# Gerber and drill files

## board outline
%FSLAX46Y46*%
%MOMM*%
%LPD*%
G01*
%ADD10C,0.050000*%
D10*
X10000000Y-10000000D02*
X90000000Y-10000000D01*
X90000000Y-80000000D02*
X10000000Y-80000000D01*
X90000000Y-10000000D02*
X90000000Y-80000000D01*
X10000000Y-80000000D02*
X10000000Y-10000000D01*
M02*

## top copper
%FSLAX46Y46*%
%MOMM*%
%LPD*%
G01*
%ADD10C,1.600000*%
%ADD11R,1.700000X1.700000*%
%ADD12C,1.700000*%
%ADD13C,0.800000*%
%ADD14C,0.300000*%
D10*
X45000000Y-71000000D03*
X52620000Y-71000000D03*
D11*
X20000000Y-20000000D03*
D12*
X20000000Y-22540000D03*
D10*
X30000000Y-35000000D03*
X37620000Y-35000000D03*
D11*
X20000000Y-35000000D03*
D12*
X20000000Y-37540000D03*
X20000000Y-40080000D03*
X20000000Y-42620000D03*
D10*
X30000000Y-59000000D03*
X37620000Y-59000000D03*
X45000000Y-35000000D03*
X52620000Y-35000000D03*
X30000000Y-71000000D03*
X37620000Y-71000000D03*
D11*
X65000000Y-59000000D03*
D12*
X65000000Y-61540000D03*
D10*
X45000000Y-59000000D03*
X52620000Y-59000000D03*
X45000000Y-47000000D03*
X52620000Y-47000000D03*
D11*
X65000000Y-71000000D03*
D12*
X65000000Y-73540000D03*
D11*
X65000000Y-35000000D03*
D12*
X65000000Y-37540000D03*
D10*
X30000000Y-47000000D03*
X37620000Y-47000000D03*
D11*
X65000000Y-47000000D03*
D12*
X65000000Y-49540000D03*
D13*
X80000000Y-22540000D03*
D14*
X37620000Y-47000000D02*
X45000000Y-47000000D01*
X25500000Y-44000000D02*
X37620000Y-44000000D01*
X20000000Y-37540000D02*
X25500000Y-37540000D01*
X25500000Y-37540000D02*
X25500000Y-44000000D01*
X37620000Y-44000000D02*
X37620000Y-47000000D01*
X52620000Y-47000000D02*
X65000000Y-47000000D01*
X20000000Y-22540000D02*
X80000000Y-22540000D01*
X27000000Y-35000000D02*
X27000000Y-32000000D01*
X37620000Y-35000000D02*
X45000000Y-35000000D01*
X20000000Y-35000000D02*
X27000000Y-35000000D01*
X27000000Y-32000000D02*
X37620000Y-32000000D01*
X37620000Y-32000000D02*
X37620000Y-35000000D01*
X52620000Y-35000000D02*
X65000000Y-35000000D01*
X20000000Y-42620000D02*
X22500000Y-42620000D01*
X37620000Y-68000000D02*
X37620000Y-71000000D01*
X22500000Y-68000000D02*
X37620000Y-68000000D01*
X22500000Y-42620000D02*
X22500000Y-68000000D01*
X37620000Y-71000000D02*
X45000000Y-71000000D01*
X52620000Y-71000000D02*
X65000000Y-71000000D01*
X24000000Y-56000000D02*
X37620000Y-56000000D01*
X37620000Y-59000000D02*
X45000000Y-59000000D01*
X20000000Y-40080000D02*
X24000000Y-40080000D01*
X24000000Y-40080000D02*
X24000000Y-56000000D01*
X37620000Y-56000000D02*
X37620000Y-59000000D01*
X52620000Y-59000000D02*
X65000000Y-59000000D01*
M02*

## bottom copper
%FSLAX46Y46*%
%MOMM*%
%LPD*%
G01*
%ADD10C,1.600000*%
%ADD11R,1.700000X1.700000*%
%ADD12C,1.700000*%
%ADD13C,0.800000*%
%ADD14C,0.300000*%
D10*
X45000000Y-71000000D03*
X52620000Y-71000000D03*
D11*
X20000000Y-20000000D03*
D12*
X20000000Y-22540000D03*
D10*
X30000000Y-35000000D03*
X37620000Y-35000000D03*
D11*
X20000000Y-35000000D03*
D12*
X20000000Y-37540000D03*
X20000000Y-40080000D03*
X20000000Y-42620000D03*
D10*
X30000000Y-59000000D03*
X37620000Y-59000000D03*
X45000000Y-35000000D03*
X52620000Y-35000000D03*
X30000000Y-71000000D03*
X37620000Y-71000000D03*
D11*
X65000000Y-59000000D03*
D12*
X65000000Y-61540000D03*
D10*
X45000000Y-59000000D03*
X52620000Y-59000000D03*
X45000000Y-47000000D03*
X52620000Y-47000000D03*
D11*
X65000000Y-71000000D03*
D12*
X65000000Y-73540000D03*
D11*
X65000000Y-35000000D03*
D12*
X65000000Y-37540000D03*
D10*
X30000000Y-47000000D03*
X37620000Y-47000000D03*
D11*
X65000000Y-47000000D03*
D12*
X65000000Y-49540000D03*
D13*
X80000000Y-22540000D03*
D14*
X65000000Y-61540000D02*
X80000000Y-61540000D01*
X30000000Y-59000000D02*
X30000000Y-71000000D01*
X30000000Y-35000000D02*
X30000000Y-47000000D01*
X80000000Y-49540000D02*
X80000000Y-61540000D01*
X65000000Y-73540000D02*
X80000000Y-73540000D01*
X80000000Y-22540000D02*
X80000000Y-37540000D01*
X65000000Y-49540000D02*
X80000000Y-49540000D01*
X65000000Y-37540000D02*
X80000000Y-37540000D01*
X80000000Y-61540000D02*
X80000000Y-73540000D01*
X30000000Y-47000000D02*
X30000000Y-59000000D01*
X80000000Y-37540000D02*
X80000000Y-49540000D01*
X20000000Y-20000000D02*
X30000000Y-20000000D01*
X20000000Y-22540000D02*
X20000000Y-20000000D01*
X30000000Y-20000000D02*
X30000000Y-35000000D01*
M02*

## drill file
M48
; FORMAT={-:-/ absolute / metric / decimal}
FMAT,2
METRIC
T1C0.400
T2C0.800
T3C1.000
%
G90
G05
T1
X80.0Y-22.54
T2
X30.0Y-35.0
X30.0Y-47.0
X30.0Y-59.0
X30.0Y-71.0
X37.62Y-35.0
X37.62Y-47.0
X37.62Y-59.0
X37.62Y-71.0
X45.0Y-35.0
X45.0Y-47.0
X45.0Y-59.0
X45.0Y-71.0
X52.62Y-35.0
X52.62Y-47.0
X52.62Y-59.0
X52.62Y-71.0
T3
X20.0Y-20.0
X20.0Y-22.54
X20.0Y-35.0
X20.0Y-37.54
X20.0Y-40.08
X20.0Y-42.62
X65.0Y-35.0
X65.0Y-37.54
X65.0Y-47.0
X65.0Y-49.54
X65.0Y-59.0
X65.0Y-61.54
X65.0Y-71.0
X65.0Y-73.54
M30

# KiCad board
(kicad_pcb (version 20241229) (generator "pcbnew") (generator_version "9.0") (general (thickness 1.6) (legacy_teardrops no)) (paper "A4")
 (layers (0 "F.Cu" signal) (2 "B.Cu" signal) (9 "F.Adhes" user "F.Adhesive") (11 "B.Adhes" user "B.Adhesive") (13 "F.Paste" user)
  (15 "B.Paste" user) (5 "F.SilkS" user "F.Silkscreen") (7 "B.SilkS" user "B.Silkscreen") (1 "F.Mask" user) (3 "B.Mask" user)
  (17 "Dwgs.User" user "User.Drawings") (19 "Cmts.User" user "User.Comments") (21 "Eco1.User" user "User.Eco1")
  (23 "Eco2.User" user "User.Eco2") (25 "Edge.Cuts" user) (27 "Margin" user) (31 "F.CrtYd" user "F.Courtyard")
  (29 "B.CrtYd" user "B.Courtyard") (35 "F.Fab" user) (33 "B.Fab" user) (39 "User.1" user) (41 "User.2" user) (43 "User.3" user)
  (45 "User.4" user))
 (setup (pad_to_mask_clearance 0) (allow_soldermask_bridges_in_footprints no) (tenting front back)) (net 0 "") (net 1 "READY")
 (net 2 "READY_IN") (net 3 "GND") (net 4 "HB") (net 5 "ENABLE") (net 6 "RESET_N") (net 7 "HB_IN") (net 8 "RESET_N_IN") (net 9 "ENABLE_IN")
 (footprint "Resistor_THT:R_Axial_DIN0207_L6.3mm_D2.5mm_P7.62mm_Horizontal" (layer "F.Cu") (at 45 71)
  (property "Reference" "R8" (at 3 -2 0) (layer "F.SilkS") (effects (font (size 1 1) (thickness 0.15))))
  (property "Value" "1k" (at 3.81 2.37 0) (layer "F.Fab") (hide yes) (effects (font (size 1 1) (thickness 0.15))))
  (pad "1" thru_hole circle (at 0 0) (size 1.6 1.6) (drill 0.8) (layers "*.Cu" "*.Mask") (remove_unused_layers no) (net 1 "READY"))
  (pad "2" thru_hole circle (at 7.62 0) (size 1.6 1.6) (drill 0.8) (layers "*.Cu" "*.Mask") (remove_unused_layers no) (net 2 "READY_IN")))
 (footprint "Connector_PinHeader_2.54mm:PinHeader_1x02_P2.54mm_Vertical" (layer "F.Cu") (at 20 20)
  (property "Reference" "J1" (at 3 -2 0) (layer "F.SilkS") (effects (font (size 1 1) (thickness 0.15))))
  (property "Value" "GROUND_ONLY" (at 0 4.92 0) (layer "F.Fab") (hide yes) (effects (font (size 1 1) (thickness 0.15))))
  (pad "1" thru_hole rect (at 0 0) (size 1.7 1.7) (drill 1) (layers "*.Cu" "*.Mask") (remove_unused_layers no) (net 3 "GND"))
  (pad "2" thru_hole circle (at 0 2.54) (size 1.7 1.7) (drill 1) (layers "*.Cu" "*.Mask") (remove_unused_layers no) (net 3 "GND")))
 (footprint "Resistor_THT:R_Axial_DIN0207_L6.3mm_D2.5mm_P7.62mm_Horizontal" (layer "F.Cu") (at 30 35)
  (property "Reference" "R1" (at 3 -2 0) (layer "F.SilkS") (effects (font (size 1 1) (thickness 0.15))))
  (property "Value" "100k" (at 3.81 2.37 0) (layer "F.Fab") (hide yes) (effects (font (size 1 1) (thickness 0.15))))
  (pad "1" thru_hole circle (at 0 0) (size 1.6 1.6) (drill 0.8) (layers "*.Cu" "*.Mask") (remove_unused_layers no) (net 3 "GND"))
  (pad "2" thru_hole circle (at 7.62 0) (size 1.6 1.6) (drill 0.8) (layers "*.Cu" "*.Mask") (remove_unused_layers no) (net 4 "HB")))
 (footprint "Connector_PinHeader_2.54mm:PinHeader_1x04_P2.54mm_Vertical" (layer "F.Cu") (at 20 35)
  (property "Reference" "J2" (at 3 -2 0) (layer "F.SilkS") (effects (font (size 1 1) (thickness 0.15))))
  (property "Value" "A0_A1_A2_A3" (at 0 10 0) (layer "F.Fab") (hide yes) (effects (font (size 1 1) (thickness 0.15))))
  (pad "1" thru_hole rect (at 0 0) (size 1.7 1.7) (drill 1) (layers "*.Cu" "*.Mask") (remove_unused_layers no) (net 4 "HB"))
  (pad "2" thru_hole circle (at 0 2.54) (size 1.7 1.7) (drill 1) (layers "*.Cu" "*.Mask") (remove_unused_layers no) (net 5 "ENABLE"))
  (pad "3" thru_hole circle (at 0 5.08) (size 1.7 1.7) (drill 1) (layers "*.Cu" "*.Mask") (remove_unused_layers no) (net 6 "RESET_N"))
  (pad "4" thru_hole circle (at 0 7.62) (size 1.7 1.7) (drill 1) (layers "*.Cu" "*.Mask") (remove_unused_layers no) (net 1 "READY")))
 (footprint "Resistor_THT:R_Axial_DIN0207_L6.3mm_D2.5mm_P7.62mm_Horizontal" (layer "F.Cu") (at 30 59)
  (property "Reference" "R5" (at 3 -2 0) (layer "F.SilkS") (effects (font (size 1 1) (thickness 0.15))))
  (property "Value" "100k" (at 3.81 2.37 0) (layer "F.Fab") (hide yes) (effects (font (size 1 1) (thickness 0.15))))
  (pad "1" thru_hole circle (at 0 0) (size 1.6 1.6) (drill 0.8) (layers "*.Cu" "*.Mask") (remove_unused_layers no) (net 3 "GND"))
  (pad "2" thru_hole circle (at 7.62 0) (size 1.6 1.6) (drill 0.8) (layers "*.Cu" "*.Mask") (remove_unused_layers no) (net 6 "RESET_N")))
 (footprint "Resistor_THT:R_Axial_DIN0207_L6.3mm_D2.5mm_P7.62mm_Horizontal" (layer "F.Cu") (at 45 35)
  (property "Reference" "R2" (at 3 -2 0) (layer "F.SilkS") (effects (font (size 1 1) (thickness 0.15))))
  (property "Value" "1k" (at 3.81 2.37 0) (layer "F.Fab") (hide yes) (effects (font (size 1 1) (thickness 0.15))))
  (pad "1" thru_hole circle (at 0 0) (size 1.6 1.6) (drill 0.8) (layers "*.Cu" "*.Mask") (remove_unused_layers no) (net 4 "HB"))
  (pad "2" thru_hole circle (at 7.62 0) (size 1.6 1.6) (drill 0.8) (layers "*.Cu" "*.Mask") (remove_unused_layers no) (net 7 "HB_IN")))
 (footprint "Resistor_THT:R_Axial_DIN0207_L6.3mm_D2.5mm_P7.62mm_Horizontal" (layer "F.Cu") (at 30 71)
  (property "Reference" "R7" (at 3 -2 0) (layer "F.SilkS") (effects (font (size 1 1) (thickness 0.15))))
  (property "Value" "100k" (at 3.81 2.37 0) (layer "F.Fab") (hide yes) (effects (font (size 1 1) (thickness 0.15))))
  (pad "1" thru_hole circle (at 0 0) (size 1.6 1.6) (drill 0.8) (layers "*.Cu" "*.Mask") (remove_unused_layers no) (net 3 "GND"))
  (pad "2" thru_hole circle (at 7.62 0) (size 1.6 1.6) (drill 0.8) (layers "*.Cu" "*.Mask") (remove_unused_layers no) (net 1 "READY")))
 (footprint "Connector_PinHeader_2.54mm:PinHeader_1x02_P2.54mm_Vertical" (layer "F.Cu") (at 65 59)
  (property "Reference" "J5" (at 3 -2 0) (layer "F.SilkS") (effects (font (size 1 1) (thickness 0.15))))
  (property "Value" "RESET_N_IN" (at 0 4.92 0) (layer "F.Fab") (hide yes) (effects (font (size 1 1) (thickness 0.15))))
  (pad "1" thru_hole rect (at 0 0) (size 1.7 1.7) (drill 1) (layers "*.Cu" "*.Mask") (remove_unused_layers no) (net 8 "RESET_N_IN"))
  (pad "2" thru_hole circle (at 0 2.54) (size 1.7 1.7) (drill 1) (layers "*.Cu" "*.Mask") (remove_unused_layers no) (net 3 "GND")))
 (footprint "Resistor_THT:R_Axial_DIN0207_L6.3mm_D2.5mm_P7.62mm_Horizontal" (layer "F.Cu") (at 45 59)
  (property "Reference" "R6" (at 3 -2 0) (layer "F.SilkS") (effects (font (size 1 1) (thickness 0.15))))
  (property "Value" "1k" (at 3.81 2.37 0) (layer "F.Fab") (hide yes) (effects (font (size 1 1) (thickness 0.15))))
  (pad "1" thru_hole circle (at 0 0) (size 1.6 1.6) (drill 0.8) (layers "*.Cu" "*.Mask") (remove_unused_layers no) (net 6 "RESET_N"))
  (pad "2" thru_hole circle (at 7.62 0) (size 1.6 1.6) (drill 0.8) (layers "*.Cu" "*.Mask") (remove_unused_layers no) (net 8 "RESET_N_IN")))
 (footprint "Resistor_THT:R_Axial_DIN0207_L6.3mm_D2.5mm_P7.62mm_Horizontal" (layer "F.Cu") (at 45 47)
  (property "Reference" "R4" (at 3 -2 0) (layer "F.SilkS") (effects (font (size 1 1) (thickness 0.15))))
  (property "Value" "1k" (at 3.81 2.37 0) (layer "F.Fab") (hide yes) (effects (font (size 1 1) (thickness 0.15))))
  (pad "1" thru_hole circle (at 0 0) (size 1.6 1.6) (drill 0.8) (layers "*.Cu" "*.Mask") (remove_unused_layers no) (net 5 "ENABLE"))
  (pad "2" thru_hole circle (at 7.62 0) (size 1.6 1.6) (drill 0.8) (layers "*.Cu" "*.Mask") (remove_unused_layers no) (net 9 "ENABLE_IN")))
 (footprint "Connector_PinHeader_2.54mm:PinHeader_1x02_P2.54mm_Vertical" (layer "F.Cu") (at 65 71)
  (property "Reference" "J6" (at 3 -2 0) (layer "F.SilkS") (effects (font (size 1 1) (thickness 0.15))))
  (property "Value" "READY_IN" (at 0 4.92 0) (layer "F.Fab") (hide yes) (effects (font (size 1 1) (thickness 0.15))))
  (pad "1" thru_hole rect (at 0 0) (size 1.7 1.7) (drill 1) (layers "*.Cu" "*.Mask") (remove_unused_layers no) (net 2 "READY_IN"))
  (pad "2" thru_hole circle (at 0 2.54) (size 1.7 1.7) (drill 1) (layers "*.Cu" "*.Mask") (remove_unused_layers no) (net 3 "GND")))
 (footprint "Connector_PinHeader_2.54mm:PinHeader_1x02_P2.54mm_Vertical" (layer "F.Cu") (at 65 35)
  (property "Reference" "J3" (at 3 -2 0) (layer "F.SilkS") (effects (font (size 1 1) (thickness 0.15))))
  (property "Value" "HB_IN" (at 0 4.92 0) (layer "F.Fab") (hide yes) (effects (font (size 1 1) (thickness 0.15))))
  (pad "1" thru_hole rect (at 0 0) (size 1.7 1.7) (drill 1) (layers "*.Cu" "*.Mask") (remove_unused_layers no) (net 7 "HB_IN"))
  (pad "2" thru_hole circle (at 0 2.54) (size 1.7 1.7) (drill 1) (layers "*.Cu" "*.Mask") (remove_unused_layers no) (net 3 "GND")))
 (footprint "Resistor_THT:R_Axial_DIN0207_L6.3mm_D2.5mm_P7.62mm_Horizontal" (layer "F.Cu") (at 30 47)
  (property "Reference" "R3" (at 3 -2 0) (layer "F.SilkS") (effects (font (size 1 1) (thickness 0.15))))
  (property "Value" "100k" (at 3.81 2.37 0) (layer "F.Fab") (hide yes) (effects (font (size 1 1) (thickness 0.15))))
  (pad "1" thru_hole circle (at 0 0) (size 1.6 1.6) (drill 0.8) (layers "*.Cu" "*.Mask") (remove_unused_layers no) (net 3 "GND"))
  (pad "2" thru_hole circle (at 7.62 0) (size 1.6 1.6) (drill 0.8) (layers "*.Cu" "*.Mask") (remove_unused_layers no) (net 5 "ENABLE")))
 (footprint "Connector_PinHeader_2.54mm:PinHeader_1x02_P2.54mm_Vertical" (layer "F.Cu") (at 65 47)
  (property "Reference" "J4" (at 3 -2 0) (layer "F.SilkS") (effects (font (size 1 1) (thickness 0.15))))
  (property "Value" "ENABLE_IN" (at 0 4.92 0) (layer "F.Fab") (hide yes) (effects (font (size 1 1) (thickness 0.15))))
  (pad "1" thru_hole rect (at 0 0) (size 1.7 1.7) (drill 1) (layers "*.Cu" "*.Mask") (remove_unused_layers no) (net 9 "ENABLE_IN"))
  (pad "2" thru_hole circle (at 0 2.54) (size 1.7 1.7) (drill 1) (layers "*.Cu" "*.Mask") (remove_unused_layers no) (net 3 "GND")))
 (gr_line (start 10 10) (end 90 10) (stroke (width 0.05) (type default)) (layer "Edge.Cuts"))
 (gr_line (start 90 80) (end 10 80) (stroke (width 0.05) (type default)) (layer "Edge.Cuts"))
 (gr_line (start 90 10) (end 90 80) (stroke (width 0.05) (type default)) (layer "Edge.Cuts"))
 (gr_line (start 10 80) (end 10 10) (stroke (width 0.05) (type default)) (layer "Edge.Cuts"))
 (segment (start 37.62 47) (end 45 47) (width 0.3) (layer "F.Cu") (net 5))
 (segment (start 25.5 44) (end 37.62 44) (width 0.3) (layer "F.Cu") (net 5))
 (segment (start 20 37.54) (end 25.5 37.54) (width 0.3) (layer "F.Cu") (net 5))
 (segment (start 25.5 37.54) (end 25.5 44) (width 0.3) (layer "F.Cu") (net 5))
 (segment (start 37.62 44) (end 37.62 47) (width 0.3) (layer "F.Cu") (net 5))
 (segment (start 52.62 47) (end 65 47) (width 0.3) (layer "F.Cu") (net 9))
 (segment (start 20 22.54) (end 80 22.54) (width 0.3) (layer "F.Cu") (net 3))
 (via (at 80 22.54) (size 0.8) (drill 0.4) (layers "F.Cu" "B.Cu") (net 3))
 (segment (start 65 61.54) (end 80 61.54) (width 0.3) (layer "B.Cu") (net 3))
 (segment (start 30 59) (end 30 71) (width 0.3) (layer "B.Cu") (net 3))
 (segment (start 30 35) (end 30 47) (width 0.3) (layer "B.Cu") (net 3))
 (segment (start 80 49.54) (end 80 61.54) (width 0.3) (layer "B.Cu") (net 3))
 (segment (start 65 73.54) (end 80 73.54) (width 0.3) (layer "B.Cu") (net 3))
 (segment (start 80 22.54) (end 80 37.54) (width 0.3) (layer "B.Cu") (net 3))
 (segment (start 65 49.54) (end 80 49.54) (width 0.3) (layer "B.Cu") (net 3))
 (segment (start 65 37.54) (end 80 37.54) (width 0.3) (layer "B.Cu") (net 3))
 (segment (start 80 61.54) (end 80 73.54) (width 0.3) (layer "B.Cu") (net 3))
 (segment (start 30 47) (end 30 59) (width 0.3) (layer "B.Cu") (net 3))
 (segment (start 80 37.54) (end 80 49.54) (width 0.3) (layer "B.Cu") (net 3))
 (segment (start 20 20) (end 30 20) (width 0.3) (layer "B.Cu") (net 3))
 (segment (start 20 22.54) (end 20 20) (width 0.3) (layer "B.Cu") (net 3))
 (segment (start 30 20) (end 30 35) (width 0.3) (layer "B.Cu") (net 3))
 (segment (start 27 35) (end 27 32) (width 0.3) (layer "F.Cu") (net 4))
 (segment (start 37.62 35) (end 45 35) (width 0.3) (layer "F.Cu") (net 4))
 (segment (start 20 35) (end 27 35) (width 0.3) (layer "F.Cu") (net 4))
 (segment (start 27 32) (end 37.62 32) (width 0.3) (layer "F.Cu") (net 4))
 (segment (start 37.62 32) (end 37.62 35) (width 0.3) (layer "F.Cu") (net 4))
 (segment (start 52.62 35) (end 65 35) (width 0.3) (layer "F.Cu") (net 7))
 (segment (start 20 42.62) (end 22.5 42.62) (width 0.3) (layer "F.Cu") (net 1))
 (segment (start 37.62 68) (end 37.62 71) (width 0.3) (layer "F.Cu") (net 1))
 (segment (start 22.5 68) (end 37.62 68) (width 0.3) (layer "F.Cu") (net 1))
 (segment (start 22.5 42.62) (end 22.5 68) (width 0.3) (layer "F.Cu") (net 1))
 (segment (start 37.62 71) (end 45 71) (width 0.3) (layer "F.Cu") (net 1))
 (segment (start 52.62 71) (end 65 71) (width 0.3) (layer "F.Cu") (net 2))
 (segment (start 24 56) (end 37.62 56) (width 0.3) (layer "F.Cu") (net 6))
 (segment (start 37.62 59) (end 45 59) (width 0.3) (layer "F.Cu") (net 6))
 (segment (start 20 40.08) (end 24 40.08) (width 0.3) (layer "F.Cu") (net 6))
 (segment (start 24 40.08) (end 24 56) (width 0.3) (layer "F.Cu") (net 6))
 (segment (start 37.62 56) (end 37.62 59) (width 0.3) (layer "F.Cu") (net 6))
 (segment (start 52.62 59) (end 65 59) (width 0.3) (layer "F.Cu") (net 8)))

